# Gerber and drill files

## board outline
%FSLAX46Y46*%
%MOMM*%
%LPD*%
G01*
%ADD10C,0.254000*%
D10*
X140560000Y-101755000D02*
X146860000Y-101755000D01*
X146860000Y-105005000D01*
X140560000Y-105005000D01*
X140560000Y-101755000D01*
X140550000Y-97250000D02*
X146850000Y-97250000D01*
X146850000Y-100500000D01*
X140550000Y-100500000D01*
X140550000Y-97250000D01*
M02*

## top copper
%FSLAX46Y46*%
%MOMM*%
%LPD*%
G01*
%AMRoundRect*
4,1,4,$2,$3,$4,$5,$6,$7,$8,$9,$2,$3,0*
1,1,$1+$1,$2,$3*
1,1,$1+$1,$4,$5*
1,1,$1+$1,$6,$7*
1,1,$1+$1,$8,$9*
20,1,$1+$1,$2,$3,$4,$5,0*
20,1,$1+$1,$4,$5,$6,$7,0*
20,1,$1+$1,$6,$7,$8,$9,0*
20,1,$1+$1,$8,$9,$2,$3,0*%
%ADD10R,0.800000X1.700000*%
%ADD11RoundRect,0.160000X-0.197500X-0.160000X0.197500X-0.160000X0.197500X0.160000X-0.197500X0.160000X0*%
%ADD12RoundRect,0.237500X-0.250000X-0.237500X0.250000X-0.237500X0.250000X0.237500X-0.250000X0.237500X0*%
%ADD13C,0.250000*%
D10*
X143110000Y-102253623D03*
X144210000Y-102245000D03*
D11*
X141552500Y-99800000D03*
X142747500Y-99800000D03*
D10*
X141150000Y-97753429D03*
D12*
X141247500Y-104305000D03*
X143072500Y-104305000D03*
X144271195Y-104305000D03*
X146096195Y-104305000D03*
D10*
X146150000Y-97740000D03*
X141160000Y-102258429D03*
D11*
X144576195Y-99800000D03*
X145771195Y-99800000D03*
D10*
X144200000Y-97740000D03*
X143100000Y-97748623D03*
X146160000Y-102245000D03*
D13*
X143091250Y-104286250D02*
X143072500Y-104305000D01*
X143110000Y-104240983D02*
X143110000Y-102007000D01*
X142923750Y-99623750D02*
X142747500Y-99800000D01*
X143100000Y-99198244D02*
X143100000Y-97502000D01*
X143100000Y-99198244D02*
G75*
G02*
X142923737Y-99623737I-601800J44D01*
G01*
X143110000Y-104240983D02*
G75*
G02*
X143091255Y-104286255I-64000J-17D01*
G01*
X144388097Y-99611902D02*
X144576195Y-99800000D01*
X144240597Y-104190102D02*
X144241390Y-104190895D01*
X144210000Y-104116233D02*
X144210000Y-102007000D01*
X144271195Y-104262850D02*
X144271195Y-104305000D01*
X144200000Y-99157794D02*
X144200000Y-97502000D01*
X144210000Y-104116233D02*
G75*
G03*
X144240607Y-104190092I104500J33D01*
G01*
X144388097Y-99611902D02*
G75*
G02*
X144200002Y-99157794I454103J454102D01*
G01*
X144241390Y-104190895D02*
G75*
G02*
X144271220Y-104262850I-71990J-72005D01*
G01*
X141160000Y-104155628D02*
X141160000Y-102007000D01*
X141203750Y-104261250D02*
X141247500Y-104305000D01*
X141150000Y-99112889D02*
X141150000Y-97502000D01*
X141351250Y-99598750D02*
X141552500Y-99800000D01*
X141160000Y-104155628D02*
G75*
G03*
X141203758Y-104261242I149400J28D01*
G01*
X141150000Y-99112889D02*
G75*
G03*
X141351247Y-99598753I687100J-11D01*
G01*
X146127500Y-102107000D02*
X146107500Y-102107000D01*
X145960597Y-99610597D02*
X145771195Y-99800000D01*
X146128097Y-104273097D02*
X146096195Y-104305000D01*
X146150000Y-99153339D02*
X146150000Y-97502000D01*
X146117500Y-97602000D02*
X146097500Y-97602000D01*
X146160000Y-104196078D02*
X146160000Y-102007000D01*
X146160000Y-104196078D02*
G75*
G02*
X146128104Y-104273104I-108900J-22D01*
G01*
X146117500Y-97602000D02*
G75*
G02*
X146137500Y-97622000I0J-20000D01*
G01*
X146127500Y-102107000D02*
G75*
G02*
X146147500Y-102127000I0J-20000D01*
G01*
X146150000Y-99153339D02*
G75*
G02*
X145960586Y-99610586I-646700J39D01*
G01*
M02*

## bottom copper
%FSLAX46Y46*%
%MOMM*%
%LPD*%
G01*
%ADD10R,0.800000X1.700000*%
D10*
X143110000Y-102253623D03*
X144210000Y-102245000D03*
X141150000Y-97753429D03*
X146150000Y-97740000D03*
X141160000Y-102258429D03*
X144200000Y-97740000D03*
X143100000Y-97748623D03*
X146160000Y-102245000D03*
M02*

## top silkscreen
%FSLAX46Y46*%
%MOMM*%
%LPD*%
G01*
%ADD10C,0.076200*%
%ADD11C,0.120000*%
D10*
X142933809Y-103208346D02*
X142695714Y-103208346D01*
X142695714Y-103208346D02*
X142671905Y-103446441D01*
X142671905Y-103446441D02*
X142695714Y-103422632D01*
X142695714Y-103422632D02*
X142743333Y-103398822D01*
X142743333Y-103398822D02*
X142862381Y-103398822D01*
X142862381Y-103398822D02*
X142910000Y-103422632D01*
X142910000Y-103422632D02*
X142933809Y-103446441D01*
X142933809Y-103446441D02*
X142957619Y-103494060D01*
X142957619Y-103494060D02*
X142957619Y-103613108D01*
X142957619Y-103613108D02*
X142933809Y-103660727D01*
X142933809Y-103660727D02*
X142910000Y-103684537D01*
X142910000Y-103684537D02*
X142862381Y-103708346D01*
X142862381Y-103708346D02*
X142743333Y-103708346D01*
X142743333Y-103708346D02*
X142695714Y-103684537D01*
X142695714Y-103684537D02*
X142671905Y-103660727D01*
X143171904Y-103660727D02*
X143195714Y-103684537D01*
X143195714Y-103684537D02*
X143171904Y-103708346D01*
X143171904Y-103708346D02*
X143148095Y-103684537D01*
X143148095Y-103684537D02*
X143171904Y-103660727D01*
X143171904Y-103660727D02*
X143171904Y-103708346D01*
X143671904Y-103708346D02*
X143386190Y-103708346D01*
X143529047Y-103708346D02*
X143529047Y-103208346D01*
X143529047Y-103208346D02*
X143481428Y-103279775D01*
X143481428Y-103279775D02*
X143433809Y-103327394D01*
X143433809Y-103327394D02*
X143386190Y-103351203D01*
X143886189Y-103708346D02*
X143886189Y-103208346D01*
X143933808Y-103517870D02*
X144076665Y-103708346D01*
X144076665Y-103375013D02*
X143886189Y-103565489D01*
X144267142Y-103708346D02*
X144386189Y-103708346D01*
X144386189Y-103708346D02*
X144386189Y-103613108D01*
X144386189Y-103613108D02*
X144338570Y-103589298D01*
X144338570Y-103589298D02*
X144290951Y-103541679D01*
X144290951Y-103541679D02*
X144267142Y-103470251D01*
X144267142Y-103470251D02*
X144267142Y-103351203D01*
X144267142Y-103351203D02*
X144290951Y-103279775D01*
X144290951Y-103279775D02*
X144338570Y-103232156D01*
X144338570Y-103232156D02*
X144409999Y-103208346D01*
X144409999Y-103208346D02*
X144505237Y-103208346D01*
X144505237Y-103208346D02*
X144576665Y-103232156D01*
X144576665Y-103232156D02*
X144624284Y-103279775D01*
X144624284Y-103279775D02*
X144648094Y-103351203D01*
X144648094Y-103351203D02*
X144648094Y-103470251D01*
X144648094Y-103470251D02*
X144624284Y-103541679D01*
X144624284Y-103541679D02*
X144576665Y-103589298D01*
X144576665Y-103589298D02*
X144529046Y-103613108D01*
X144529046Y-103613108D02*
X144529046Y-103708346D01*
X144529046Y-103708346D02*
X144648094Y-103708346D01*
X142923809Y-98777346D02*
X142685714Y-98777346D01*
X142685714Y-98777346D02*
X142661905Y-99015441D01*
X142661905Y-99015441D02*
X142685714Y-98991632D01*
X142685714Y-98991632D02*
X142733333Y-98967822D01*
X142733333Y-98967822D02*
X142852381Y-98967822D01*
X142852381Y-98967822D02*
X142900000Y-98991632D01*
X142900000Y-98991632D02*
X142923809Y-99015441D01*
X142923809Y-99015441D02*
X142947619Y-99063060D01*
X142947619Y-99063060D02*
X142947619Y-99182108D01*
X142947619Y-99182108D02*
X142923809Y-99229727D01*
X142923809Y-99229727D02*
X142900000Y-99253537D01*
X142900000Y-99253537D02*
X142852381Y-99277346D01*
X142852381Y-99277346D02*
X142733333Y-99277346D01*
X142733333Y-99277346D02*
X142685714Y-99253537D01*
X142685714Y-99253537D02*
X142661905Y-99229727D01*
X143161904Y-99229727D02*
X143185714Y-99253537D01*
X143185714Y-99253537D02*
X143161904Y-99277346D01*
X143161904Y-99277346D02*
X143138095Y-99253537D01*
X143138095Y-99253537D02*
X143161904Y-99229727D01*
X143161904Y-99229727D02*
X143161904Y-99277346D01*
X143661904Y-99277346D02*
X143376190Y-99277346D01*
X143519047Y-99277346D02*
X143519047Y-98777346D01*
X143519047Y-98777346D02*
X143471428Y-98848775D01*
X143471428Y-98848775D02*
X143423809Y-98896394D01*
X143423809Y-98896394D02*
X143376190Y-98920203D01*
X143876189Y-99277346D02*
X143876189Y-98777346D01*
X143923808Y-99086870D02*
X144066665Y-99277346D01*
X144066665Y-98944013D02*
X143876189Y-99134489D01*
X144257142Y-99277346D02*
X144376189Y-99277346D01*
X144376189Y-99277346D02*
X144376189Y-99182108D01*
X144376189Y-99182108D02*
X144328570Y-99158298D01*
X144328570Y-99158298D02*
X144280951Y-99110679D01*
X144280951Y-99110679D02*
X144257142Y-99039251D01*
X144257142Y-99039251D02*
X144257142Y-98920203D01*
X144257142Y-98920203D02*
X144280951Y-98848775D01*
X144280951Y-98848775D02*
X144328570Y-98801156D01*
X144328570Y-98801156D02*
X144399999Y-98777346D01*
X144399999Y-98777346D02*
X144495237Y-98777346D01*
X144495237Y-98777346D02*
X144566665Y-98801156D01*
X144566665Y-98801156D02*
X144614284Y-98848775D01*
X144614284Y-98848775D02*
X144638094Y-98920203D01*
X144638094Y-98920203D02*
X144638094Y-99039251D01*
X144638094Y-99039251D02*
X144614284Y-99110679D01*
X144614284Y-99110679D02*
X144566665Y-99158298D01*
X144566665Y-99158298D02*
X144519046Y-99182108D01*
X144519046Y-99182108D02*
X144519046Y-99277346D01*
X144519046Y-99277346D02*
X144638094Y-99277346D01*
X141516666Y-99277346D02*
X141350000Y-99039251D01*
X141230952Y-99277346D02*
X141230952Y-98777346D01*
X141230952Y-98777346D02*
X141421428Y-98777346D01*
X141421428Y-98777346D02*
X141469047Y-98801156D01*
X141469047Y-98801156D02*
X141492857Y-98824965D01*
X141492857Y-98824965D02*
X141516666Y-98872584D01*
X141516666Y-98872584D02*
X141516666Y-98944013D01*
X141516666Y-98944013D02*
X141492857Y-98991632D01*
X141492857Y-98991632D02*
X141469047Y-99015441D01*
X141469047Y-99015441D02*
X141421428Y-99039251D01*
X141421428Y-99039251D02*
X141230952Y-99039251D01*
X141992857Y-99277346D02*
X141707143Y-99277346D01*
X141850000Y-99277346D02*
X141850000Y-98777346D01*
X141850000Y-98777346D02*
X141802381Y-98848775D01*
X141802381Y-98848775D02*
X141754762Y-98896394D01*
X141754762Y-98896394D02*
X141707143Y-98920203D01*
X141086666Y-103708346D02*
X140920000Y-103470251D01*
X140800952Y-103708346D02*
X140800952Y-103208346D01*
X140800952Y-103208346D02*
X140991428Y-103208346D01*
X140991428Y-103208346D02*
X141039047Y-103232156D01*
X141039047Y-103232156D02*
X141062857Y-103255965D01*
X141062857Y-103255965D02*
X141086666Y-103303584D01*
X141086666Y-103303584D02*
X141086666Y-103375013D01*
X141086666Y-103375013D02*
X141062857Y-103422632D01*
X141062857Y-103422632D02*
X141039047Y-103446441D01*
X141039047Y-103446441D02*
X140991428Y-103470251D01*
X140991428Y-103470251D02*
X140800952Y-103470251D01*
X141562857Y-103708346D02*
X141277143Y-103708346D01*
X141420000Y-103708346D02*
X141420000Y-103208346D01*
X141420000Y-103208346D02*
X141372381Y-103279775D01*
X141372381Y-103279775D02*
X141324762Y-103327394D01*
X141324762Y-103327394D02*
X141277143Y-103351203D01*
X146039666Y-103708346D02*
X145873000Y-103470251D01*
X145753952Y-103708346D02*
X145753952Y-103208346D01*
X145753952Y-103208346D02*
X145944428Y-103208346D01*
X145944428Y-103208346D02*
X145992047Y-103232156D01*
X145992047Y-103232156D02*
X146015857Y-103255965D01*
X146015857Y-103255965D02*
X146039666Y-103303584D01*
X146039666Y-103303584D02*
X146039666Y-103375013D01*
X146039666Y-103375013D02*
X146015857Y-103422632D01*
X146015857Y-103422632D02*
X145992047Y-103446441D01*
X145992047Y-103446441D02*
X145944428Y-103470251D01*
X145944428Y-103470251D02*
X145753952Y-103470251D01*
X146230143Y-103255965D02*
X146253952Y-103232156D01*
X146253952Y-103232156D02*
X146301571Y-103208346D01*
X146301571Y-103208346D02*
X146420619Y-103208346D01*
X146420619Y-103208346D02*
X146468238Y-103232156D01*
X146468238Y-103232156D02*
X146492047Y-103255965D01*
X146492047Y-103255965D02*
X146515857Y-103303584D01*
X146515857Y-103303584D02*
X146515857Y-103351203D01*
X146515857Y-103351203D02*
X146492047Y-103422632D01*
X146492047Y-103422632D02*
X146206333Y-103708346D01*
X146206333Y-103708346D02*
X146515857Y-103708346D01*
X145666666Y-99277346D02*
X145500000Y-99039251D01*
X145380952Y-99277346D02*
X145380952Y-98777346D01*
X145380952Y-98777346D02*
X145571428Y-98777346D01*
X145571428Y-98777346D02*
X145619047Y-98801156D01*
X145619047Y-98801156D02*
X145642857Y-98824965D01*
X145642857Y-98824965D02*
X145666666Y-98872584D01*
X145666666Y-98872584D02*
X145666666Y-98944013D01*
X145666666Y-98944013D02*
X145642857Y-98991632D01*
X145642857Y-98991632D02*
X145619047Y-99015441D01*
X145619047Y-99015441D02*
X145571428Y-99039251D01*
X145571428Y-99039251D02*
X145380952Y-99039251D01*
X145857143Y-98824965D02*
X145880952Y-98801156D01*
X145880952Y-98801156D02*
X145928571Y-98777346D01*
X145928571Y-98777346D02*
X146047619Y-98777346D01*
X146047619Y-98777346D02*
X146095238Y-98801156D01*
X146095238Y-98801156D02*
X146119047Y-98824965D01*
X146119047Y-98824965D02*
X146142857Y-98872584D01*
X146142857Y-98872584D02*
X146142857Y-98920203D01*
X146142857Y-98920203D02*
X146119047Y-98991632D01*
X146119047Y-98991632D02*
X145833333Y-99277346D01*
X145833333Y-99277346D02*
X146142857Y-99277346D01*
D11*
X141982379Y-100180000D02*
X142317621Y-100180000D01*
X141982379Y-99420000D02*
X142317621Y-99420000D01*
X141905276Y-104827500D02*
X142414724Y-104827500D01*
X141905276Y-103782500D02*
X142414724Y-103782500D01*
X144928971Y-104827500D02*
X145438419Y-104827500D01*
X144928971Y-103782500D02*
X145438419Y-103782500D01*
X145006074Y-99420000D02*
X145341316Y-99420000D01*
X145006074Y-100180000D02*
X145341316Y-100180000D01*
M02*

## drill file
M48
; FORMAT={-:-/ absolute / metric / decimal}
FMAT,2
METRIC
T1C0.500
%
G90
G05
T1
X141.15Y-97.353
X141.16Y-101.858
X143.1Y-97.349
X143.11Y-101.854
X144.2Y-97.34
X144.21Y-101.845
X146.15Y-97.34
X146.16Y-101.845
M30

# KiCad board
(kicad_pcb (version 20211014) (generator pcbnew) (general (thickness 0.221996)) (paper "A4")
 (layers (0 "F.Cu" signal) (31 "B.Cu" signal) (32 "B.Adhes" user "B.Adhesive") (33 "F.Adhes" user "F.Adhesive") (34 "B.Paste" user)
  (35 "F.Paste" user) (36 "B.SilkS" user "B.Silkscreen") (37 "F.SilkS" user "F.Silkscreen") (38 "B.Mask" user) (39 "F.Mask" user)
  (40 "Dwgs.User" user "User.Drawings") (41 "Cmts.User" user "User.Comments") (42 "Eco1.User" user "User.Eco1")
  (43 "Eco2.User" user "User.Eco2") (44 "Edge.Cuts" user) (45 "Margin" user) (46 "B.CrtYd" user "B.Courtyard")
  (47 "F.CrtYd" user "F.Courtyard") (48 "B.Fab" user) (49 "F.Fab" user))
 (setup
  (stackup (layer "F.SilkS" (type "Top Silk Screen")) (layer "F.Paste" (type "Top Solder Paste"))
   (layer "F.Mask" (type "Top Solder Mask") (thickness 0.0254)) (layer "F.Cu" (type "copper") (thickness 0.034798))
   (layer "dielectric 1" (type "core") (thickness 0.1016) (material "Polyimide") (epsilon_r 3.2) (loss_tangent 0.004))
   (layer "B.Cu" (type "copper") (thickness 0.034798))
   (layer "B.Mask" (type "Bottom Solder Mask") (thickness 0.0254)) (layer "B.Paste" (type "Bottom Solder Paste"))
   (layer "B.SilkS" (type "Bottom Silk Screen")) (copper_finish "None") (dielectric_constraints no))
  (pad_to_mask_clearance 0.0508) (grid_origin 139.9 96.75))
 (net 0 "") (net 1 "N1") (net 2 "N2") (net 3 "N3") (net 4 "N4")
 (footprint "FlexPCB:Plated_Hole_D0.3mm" (layer "F.Cu") (at 145.41 103.123623 -90)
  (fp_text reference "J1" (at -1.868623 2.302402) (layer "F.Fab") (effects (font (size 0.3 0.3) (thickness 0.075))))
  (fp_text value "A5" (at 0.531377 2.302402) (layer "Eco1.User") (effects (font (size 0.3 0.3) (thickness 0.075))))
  (pad "1" thru_hole rect (at -1.27 2.3 270) (size 1.7 0.8) (drill 0.5 (offset 0.4 0)) (layers *.Cu *.Mask) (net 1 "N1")))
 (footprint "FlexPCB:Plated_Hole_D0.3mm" (layer "F.Cu") (at 146.51 103.115 -90)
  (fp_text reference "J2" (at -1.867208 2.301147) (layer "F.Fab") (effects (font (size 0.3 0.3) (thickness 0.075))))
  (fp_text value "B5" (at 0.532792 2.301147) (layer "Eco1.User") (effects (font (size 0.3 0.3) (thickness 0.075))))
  (pad "1" thru_hole rect (at -1.27 2.3 270) (size 1.7 0.8) (drill 0.5 (offset 0.4 0)) (layers *.Cu *.Mask) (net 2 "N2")))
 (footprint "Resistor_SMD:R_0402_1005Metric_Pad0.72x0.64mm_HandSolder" (layer "F.Cu") (at 142.15 99.8)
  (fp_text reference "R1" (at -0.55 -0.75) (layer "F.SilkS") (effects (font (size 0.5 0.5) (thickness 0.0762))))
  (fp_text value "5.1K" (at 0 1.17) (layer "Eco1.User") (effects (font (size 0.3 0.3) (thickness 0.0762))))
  (fp_line (start -0.167621 0.38) (end 0.167621 0.38) (layer "F.SilkS") (width 0.12))
  (fp_line (start -0.167621 -0.38) (end 0.167621 -0.38) (layer "F.SilkS") (width 0.12))
  (pad "1" smd roundrect (at -0.5975 0) (size 0.715 0.64) (layers "F.Cu" "F.Paste" "F.Mask") (roundrect_rratio 0.25) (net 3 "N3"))
  (pad "2" smd roundrect (at 0.5975 0) (size 0.715 0.64) (layers "F.Cu" "F.Paste" "F.Mask") (roundrect_rratio 0.25) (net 1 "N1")))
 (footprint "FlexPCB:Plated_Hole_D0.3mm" (layer "F.Cu") (at 143.45 98.623429 -90)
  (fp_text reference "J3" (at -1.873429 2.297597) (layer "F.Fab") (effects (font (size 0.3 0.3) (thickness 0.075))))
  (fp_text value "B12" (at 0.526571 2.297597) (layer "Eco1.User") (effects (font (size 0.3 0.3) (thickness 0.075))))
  (pad "1" thru_hole rect (at -1.27 2.3 270) (size 1.7 0.8) (drill 0.5 (offset 0.4 0)) (layers *.Cu *.Mask) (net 3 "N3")))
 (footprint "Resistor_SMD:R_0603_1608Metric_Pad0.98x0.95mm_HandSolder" (layer "F.Cu") (at 142.16 104.305)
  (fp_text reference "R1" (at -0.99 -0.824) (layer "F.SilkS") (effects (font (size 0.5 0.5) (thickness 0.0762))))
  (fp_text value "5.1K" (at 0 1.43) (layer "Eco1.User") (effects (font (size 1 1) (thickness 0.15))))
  (fp_line (start -0.254724 0.5225) (end 0.254724 0.5225) (layer "F.SilkS") (width 0.12))
  (fp_line (start -0.254724 -0.5225) (end 0.254724 -0.5225) (layer "F.SilkS") (width 0.12))
  (pad "1" smd roundrect (at -0.9125 0) (size 0.975 0.95) (layers "F.Cu" "F.Paste" "F.Mask") (roundrect_rratio 0.25) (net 3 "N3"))
  (pad "2" smd roundrect (at 0.9125 0) (size 0.975 0.95) (layers "F.Cu" "F.Paste" "F.Mask") (roundrect_rratio 0.25) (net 1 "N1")))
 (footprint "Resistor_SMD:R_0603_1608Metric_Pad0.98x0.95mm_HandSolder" (layer "F.Cu") (at 145.183695 104.305)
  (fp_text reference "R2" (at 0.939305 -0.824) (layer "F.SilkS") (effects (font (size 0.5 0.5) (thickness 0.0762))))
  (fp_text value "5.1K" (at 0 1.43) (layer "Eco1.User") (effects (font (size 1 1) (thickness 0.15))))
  (fp_line (start -0.254724 0.5225) (end 0.254724 0.5225) (layer "F.SilkS") (width 0.12))
  (fp_line (start -0.254724 -0.5225) (end 0.254724 -0.5225) (layer "F.SilkS") (width 0.12))
  (pad "1" smd roundrect (at -0.9125 0) (size 0.975 0.95) (layers "F.Cu" "F.Paste" "F.Mask") (roundrect_rratio 0.25) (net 2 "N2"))
  (pad "2" smd roundrect (at 0.9125 0) (size 0.975 0.95) (layers "F.Cu" "F.Paste" "F.Mask") (roundrect_rratio 0.25) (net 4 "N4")))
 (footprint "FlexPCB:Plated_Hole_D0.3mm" (layer "F.Cu") (at 148.45 98.61 -90)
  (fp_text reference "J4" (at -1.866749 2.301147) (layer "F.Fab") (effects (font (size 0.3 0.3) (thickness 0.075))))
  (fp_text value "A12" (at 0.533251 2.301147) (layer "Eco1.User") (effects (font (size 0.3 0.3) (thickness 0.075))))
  (pad "1" thru_hole rect (at -1.27 2.3 270) (size 1.7 0.8) (drill 0.5 (offset 0.4 0)) (layers *.Cu *.Mask) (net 4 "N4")))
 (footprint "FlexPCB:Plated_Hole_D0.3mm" (layer "F.Cu") (at 143.46 103.128429 -90)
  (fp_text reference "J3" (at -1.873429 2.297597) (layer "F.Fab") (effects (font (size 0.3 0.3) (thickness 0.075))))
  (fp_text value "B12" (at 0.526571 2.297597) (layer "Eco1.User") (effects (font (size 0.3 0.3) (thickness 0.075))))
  (pad "1" thru_hole rect (at -1.27 2.3 270) (size 1.7 0.8) (drill 0.5 (offset 0.4 0)) (layers *.Cu *.Mask) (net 3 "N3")))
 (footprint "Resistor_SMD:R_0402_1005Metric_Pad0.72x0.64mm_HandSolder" (layer "F.Cu") (at 145.173695 99.8)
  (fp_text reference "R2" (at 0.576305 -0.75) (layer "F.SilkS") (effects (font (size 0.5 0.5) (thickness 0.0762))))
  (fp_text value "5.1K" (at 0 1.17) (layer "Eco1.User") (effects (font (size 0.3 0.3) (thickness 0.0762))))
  (fp_line (start -0.167621 -0.38) (end 0.167621 -0.38) (layer "F.SilkS") (width 0.12))
  (fp_line (start -0.167621 0.38) (end 0.167621 0.38) (layer "F.SilkS") (width 0.12))
  (pad "1" smd roundrect (at -0.5975 0) (size 0.715 0.64) (layers "F.Cu" "F.Paste" "F.Mask") (roundrect_rratio 0.25) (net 2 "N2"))
  (pad "2" smd roundrect (at 0.5975 0) (size 0.715 0.64) (layers "F.Cu" "F.Paste" "F.Mask") (roundrect_rratio 0.25) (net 4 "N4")))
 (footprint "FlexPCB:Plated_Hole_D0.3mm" (layer "F.Cu") (at 146.5 98.61 -90)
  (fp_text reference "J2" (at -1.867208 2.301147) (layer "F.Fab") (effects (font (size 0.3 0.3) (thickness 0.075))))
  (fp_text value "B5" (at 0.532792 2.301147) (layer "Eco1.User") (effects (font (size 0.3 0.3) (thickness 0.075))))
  (pad "1" thru_hole rect (at -1.27 2.3 270) (size 1.7 0.8) (drill 0.5 (offset 0.4 0)) (layers *.Cu *.Mask) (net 2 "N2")))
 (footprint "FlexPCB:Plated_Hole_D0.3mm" (layer "F.Cu") (at 145.4 98.618623 -90)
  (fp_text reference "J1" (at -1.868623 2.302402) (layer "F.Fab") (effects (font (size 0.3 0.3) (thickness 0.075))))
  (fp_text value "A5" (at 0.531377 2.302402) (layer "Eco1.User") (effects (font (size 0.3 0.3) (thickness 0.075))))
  (pad "1" thru_hole rect (at -1.27 2.3 270) (size 1.7 0.8) (drill 0.5 (offset 0.4 0)) (layers *.Cu *.Mask) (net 1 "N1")))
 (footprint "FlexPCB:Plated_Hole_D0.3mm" (layer "F.Cu") (at 148.46 103.115 -90)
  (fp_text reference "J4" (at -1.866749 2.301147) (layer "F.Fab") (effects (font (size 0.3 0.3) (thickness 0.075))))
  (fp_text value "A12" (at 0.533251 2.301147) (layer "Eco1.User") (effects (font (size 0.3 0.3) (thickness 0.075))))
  (pad "1" thru_hole rect (at -1.27 2.3 270) (size 1.7 0.8) (drill 0.5 (offset 0.4 0)) (layers *.Cu *.Mask) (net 4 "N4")))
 (gr_rect (start 146.86 101.755) (end 140.56 105.005) (layer "Edge.Cuts") (width 0.254) (fill none))
 (gr_rect (start 146.85 97.25) (end 140.55 100.5) (layer "Edge.Cuts") (width 0.254) (fill none))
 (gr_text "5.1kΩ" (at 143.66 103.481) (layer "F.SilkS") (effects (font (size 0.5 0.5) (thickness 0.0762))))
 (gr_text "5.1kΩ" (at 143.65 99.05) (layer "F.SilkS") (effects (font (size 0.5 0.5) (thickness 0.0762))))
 (segment (start 143.09125 104.28625) (end 143.0725 104.305) (width 0.25) (layer "F.Cu") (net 1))
 (segment (start 143.11 104.240983) (end 143.11 102.007) (width 0.25) (layer "F.Cu") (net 1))
 (segment (start 142.92375 99.62375) (end 142.7475 99.8) (width 0.25) (layer "F.Cu") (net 1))
 (segment (start 143.1 99.198244) (end 143.1 97.502) (width 0.25) (layer "F.Cu") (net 1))
 (arc (start 143.1 99.198244) (mid 143.054194 99.428526) (end 142.92375 99.62375) (width 0.25) (layer "F.Cu") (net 1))
 (arc (start 143.11 104.240983) (mid 143.105127 104.265481) (end 143.09125 104.28625) (width 0.25) (layer "F.Cu") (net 1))
 (segment (start 144.388097 99.611902) (end 144.576195 99.8) (width 0.25) (layer "F.Cu") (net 2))
 (segment (start 144.240597 104.190102) (end 144.24139 104.190895) (width 0.25) (layer "F.Cu") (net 2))
 (segment (start 144.21 104.116233) (end 144.21 102.007) (width 0.25) (layer "F.Cu") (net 2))
 (segment (start 144.271195 104.26285) (end 144.271195 104.305) (width 0.25) (layer "F.Cu") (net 2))
 (segment (start 144.2 99.157794) (end 144.2 97.502) (width 0.25) (layer "F.Cu") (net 2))
 (arc (start 144.21 104.116233) (mid 144.217951 104.15621) (end 144.240597 104.190102) (width 0.25) (layer "F.Cu") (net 2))
 (arc (start 144.388097 99.611902) (mid 144.248884 99.403555) (end 144.2 99.157794) (width 0.25) (layer "F.Cu") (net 2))
 (arc (start 144.24139 104.190895) (mid 144.263448 104.223908) (end 144.271195 104.26285) (width 0.25) (layer "F.Cu") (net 2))
 (segment (start 141.16 104.155628) (end 141.16 102.007) (width 0.25) (layer "F.Cu") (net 3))
 (segment (start 141.20375 104.26125) (end 141.2475 104.305) (width 0.25) (layer "F.Cu") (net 3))
 (segment (start 141.15 99.112889) (end 141.15 97.502) (width 0.25) (layer "F.Cu") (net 3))
 (segment (start 141.35125 99.59875) (end 141.5525 99.8) (width 0.25) (layer "F.Cu") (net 3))
 (arc (start 141.16 104.155628) (mid 141.17137 104.21279) (end 141.20375 104.26125) (width 0.25) (layer "F.Cu") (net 3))
 (arc (start 141.15 99.112889) (mid 141.202303 99.375835) (end 141.35125 99.59875) (width 0.25) (layer "F.Cu") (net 3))
 (segment (start 146.1275 102.107) (end 146.1075 102.107) (width 0.25) (layer "F.Cu") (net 4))
 (segment (start 145.960597 99.610597) (end 145.771195 99.8) (width 0.25) (layer "F.Cu") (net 4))
 (segment (start 146.128097 104.273097) (end 146.096195 104.305) (width 0.25) (layer "F.Cu") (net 4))
 (segment (start 146.15 99.153339) (end 146.15 97.502) (width 0.25) (layer "F.Cu") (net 4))
 (segment (start 146.1175 97.602) (end 146.0975 97.602) (width 0.25) (layer "F.Cu") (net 4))
 (segment (start 146.16 104.196078) (end 146.16 102.007) (width 0.25) (layer "F.Cu") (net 4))
 (arc (start 146.16 104.196078) (mid 146.151708 104.23776) (end 146.128097 104.273097) (width 0.25) (layer "F.Cu") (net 4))
 (arc (start 146.1175 97.602) (mid 146.131642 97.607857) (end 146.1375 97.622) (width 0.25) (layer "F.Cu") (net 4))
 (arc (start 146.1275 102.107) (mid 146.141642 102.112857) (end 146.1475 102.127) (width 0.25) (layer "F.Cu") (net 4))
 (arc (start 146.15 99.153339) (mid 146.100775 99.400805) (end 145.960597 99.610597) (width 0.25) (layer "F.Cu") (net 4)))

